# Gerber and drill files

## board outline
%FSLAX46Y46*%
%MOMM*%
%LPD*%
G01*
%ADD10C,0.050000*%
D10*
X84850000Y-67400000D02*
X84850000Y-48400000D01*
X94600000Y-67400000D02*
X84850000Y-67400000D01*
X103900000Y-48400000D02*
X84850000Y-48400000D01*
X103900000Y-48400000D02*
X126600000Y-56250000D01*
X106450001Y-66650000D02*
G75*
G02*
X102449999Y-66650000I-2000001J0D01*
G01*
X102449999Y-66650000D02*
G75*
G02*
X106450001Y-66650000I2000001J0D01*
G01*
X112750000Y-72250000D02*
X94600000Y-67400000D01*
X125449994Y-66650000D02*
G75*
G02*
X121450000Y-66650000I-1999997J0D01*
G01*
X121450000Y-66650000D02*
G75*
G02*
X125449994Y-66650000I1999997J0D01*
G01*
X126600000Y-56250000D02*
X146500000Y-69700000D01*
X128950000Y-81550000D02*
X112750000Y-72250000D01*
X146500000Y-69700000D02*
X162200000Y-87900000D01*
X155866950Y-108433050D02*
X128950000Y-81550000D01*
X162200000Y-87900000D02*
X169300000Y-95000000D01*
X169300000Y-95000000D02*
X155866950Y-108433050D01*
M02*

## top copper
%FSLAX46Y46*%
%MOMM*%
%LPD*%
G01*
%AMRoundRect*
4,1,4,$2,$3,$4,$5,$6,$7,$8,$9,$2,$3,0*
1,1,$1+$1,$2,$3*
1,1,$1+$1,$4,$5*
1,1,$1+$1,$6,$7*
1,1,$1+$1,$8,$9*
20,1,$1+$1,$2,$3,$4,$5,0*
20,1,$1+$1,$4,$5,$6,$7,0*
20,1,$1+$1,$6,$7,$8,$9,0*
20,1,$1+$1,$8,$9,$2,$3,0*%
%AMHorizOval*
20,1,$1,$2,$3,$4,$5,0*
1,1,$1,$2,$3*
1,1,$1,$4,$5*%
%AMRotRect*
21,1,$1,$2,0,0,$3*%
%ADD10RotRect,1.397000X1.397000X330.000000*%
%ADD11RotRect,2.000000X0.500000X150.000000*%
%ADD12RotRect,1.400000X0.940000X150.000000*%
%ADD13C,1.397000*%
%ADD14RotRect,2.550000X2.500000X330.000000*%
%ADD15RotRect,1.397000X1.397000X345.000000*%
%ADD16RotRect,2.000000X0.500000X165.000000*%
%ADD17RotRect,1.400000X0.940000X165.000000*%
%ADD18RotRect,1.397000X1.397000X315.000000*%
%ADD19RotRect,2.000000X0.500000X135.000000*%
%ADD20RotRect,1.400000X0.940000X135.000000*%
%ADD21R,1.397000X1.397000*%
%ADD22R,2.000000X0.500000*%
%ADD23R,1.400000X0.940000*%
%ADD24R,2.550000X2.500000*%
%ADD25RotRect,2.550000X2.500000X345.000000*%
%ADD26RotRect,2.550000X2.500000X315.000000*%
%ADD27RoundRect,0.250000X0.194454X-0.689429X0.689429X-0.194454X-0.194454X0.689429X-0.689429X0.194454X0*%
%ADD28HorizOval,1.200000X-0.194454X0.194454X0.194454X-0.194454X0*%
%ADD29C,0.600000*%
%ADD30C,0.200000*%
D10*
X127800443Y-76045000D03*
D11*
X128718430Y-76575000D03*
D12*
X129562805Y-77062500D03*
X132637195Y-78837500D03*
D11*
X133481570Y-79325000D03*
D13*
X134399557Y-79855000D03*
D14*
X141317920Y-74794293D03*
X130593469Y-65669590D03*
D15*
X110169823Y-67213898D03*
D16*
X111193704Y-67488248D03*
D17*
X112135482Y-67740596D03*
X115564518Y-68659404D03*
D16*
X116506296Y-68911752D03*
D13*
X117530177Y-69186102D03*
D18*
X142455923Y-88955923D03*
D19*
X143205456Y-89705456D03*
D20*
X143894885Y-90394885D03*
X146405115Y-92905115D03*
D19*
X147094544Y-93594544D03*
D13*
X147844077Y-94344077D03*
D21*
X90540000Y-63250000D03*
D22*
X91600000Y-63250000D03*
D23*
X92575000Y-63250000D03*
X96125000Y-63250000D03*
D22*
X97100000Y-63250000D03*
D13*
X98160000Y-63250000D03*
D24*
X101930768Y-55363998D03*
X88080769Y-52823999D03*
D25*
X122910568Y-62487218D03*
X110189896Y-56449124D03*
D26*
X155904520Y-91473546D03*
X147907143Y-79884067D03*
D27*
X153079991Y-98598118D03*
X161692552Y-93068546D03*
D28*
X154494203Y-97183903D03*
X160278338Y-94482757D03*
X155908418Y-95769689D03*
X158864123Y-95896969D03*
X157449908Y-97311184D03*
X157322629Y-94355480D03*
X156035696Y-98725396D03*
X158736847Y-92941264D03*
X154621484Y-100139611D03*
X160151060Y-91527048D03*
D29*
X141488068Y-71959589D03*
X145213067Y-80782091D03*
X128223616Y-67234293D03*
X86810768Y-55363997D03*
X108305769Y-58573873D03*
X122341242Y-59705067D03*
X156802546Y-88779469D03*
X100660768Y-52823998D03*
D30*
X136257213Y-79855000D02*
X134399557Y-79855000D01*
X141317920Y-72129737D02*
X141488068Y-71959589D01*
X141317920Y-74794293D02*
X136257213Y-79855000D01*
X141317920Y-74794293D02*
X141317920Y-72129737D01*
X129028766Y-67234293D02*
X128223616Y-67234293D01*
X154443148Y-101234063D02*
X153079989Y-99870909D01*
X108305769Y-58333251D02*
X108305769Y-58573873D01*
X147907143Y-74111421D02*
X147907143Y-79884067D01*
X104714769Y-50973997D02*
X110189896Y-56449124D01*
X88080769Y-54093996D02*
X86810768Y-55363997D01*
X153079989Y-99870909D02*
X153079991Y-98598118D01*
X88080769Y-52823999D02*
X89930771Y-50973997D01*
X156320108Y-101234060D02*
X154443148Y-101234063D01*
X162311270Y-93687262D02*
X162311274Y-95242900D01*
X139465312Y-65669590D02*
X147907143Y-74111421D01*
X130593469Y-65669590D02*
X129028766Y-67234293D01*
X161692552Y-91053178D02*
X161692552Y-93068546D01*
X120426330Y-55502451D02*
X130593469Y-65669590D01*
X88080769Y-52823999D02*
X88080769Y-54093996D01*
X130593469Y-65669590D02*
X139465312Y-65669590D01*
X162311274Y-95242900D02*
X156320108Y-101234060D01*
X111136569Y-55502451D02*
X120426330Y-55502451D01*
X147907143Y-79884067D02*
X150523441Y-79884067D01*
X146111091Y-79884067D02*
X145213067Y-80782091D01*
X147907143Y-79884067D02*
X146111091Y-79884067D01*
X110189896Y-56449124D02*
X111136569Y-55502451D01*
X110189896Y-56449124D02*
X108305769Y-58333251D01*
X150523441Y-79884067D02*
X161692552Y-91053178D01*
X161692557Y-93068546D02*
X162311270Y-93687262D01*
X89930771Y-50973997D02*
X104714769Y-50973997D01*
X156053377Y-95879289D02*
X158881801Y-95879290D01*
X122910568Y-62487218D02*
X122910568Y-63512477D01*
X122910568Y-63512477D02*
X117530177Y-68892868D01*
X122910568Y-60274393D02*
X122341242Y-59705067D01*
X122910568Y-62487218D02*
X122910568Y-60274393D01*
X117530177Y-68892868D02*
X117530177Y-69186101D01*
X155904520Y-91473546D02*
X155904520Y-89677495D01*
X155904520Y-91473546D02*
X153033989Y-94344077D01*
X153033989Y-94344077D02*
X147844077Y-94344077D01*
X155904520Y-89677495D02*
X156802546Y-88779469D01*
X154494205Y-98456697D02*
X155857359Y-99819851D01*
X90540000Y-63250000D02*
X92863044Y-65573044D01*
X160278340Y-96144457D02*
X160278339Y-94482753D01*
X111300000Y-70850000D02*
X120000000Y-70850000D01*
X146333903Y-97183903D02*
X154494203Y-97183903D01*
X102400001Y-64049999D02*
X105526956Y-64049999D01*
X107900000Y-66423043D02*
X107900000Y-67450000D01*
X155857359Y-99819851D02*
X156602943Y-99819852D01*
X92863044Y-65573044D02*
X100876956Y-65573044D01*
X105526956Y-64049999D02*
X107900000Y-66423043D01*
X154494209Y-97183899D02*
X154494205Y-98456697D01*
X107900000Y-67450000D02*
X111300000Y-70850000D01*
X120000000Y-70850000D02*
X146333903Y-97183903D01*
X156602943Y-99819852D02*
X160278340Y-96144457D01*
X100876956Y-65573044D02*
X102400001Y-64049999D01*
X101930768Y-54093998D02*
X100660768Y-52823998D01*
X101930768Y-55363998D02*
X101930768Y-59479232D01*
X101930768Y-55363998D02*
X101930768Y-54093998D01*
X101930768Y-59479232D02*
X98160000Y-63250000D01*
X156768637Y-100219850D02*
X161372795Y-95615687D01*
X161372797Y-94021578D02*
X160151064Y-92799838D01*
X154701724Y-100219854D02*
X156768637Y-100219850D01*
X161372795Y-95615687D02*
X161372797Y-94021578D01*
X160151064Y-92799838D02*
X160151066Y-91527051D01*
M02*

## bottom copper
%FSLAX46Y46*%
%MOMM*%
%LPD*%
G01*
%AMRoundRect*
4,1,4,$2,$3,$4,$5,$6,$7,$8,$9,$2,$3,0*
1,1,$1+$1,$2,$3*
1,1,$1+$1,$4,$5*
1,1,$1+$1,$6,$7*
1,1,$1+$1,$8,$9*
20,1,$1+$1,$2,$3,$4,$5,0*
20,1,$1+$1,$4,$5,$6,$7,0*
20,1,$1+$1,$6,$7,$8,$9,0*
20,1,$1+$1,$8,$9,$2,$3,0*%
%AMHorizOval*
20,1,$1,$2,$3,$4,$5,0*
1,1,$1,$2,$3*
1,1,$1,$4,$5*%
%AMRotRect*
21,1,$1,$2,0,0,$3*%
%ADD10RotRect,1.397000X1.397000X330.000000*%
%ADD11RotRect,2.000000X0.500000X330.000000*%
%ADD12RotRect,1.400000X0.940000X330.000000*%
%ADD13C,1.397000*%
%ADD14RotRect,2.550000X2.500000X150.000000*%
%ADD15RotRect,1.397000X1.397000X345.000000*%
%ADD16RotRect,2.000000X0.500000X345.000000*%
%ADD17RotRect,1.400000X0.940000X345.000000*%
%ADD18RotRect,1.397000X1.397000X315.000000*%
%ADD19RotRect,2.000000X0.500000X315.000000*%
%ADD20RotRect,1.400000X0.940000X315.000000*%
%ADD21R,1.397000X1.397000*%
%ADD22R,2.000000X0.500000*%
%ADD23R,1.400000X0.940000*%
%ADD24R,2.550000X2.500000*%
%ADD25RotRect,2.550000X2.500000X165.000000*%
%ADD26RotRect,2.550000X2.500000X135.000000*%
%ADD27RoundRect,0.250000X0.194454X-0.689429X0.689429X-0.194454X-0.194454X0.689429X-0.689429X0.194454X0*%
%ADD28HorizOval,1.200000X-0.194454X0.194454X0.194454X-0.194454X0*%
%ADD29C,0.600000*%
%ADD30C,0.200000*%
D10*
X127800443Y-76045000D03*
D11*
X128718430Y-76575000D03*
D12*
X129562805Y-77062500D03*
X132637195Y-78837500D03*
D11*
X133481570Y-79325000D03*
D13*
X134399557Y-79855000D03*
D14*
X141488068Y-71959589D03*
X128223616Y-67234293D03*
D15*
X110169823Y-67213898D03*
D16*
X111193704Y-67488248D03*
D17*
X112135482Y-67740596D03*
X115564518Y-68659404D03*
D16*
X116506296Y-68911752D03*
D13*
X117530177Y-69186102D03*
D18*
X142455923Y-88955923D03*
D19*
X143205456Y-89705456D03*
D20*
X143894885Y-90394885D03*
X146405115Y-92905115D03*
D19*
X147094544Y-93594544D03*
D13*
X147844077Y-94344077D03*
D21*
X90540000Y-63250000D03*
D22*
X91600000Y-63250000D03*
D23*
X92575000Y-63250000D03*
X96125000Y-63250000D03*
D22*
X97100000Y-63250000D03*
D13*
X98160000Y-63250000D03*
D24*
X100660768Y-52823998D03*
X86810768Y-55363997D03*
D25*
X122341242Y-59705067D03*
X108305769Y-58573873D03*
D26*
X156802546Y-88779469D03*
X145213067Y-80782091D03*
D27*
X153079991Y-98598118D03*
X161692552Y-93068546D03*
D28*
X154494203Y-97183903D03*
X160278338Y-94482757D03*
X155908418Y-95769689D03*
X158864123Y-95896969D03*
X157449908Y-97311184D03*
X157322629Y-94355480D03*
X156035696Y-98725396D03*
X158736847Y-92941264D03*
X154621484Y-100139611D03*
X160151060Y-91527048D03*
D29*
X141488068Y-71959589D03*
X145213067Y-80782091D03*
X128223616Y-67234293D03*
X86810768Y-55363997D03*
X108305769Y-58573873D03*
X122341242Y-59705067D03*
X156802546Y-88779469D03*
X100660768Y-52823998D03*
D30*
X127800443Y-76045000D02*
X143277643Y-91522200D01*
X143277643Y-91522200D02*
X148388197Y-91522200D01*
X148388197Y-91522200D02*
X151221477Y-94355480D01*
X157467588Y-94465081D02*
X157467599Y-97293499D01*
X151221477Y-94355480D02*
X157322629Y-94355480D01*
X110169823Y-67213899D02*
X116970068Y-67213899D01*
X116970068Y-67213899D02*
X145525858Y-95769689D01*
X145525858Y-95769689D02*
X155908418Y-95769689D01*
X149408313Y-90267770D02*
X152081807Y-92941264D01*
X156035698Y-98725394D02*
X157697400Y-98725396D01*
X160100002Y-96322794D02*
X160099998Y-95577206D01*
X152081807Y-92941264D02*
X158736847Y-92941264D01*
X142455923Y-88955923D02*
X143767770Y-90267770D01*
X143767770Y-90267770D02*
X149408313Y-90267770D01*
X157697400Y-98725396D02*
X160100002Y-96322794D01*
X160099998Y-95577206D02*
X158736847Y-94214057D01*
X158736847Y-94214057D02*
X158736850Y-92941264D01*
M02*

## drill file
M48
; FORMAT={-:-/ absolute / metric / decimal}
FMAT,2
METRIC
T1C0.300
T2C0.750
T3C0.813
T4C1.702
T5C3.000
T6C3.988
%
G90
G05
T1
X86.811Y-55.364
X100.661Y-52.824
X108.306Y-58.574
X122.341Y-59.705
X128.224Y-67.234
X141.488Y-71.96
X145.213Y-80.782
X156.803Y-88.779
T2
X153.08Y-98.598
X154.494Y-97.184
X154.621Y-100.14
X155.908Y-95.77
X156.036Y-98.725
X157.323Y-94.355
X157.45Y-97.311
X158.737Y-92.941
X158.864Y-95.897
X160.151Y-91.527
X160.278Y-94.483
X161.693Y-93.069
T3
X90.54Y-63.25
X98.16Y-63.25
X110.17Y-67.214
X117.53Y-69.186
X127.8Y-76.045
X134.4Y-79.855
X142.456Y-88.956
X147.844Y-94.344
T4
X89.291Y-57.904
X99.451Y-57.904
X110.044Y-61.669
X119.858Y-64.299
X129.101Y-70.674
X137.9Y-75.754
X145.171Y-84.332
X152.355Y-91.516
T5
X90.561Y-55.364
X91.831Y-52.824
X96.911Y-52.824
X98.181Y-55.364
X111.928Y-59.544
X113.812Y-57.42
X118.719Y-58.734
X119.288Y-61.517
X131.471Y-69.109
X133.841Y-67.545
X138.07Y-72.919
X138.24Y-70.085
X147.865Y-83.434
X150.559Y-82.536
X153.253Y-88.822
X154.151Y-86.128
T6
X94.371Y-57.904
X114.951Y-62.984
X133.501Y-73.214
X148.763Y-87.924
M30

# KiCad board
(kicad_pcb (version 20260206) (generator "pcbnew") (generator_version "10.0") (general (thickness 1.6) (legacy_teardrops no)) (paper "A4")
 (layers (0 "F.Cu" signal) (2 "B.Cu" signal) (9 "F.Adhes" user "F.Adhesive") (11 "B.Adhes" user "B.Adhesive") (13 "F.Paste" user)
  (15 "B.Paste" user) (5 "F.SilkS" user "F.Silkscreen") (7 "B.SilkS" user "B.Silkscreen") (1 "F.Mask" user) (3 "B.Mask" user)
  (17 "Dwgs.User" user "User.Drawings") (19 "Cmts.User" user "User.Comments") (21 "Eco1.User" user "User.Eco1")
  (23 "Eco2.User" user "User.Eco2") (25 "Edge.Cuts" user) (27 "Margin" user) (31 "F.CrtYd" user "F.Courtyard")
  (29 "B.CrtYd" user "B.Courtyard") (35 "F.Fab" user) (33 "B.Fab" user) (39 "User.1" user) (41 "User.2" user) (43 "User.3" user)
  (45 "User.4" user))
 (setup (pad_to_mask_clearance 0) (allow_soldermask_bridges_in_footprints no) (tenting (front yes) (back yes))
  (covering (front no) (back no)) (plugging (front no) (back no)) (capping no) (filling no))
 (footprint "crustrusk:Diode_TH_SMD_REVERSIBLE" (layer "F.Cu") (at 131.1 77.95 -30)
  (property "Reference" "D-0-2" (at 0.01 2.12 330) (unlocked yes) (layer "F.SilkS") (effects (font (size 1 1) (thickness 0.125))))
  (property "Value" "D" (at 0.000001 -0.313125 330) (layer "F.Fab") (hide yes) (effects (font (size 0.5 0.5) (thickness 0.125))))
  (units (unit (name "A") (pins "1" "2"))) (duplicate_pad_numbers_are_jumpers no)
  (pad "1" thru_hole rect (at -3.81 0 330) (size 1.397 1.397) (drill 0.8128) (layers "*.Cu" "*.Mask") (remove_unused_layers no)
   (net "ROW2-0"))
  (pad "1" smd rect (at -2.75 0 150) (size 2 0.5) (layers "F.Cu") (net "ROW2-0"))
  (pad "1" smd rect (at -2.75 0 330) (size 2 0.5) (layers "B.Cu") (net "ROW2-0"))
  (pad "1" smd rect (at -1.775 0 150) (size 1.4 0.94) (layers "F.Cu" "F.Mask" "F.Paste") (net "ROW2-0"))
  (pad "1" smd rect (at -1.775 0 330) (size 1.4 0.94) (layers "B.Cu" "B.Mask" "B.Paste") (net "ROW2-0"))
  (pad "2" smd rect (at 1.775 0 150) (size 1.4 0.94) (layers "F.Cu" "F.Mask" "F.Paste") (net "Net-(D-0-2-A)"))
  (pad "2" smd rect (at 1.775 0 330) (size 1.4 0.94) (layers "B.Cu" "B.Mask" "B.Paste") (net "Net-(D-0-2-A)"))
  (pad "2" smd rect (at 2.75 0 150) (size 2 0.5) (layers "F.Cu") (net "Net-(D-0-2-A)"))
  (pad "2" smd rect (at 2.75 0 330) (size 2 0.5) (layers "B.Cu") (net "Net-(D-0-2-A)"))
  (pad "2" thru_hole circle (at 3.81 0 330) (size 1.397 1.397) (drill 0.8128) (layers "*.Cu" "*.Mask") (remove_unused_layers no)
   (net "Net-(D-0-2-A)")))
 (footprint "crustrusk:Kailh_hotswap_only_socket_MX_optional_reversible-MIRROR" (layer "F.Cu") (at 133.500768 73.213998 -30)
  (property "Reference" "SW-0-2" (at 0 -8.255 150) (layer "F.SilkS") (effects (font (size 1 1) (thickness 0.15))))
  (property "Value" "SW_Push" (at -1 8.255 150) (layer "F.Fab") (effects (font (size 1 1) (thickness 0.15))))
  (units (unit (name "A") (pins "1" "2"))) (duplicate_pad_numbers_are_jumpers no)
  (pad "" np_thru_hole circle (at -5.08 0 330) (size 1.7018 1.7018) (drill 1.7018) (layers "*.Cu" "*.Mask"))
  (pad "" np_thru_hole circle (at -3.81 -2.54 150) (size 3 3) (drill 3) (layers "*.Cu" "*.Mask"))
  (pad "" np_thru_hole circle (at -2.54 -5.079997 330) (size 3 3) (drill 3) (layers "*.Cu" "*.Mask"))
  (pad "" np_thru_hole circle (at 0 0 330) (size 3.9878 3.9878) (drill 3.9878) (layers "*.Cu" "*.Mask"))
  (pad "" np_thru_hole circle (at 2.540002 -5.080001 150) (size 3 3) (drill 3) (layers "*.Cu" "*.Mask"))
  (pad "" np_thru_hole circle (at 3.81 -2.540001 330) (size 3 3) (drill 3) (layers "*.Cu" "*.Mask"))
  (pad "" np_thru_hole circle (at 5.08 0 330) (size 1.7018 1.7018) (drill 1.7018) (layers "*.Cu" "*.Mask"))
  (pad "1" smd rect (at 6.29 -5.08 150) (size 2.55 2.5) (layers "B.Cu" "B.Mask" "B.Paste") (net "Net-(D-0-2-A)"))
  (pad "1" smd rect (at 7.56 -2.54 330) (size 2.55 2.5) (layers "F.Cu" "F.Mask" "F.Paste") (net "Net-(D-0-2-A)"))
  (pad "2" smd rect (at -7.56 -2.54 150) (size 2.55 2.5) (layers "B.Cu" "B.Mask" "B.Paste") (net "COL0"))
  (pad "2" smd rect (at -6.289999 -5.079999 330) (size 2.55 2.5) (layers "F.Cu" "F.Mask" "F.Paste") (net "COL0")))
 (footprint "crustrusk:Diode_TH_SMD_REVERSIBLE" (layer "F.Cu") (at 113.85 68.2 -15)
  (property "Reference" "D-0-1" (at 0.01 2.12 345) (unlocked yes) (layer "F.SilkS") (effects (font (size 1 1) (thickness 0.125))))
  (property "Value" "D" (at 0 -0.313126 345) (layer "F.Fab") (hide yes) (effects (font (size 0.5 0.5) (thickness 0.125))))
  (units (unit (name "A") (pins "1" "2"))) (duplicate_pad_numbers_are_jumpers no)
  (pad "1" thru_hole rect (at -3.81 -0.000001 345) (size 1.397 1.397) (drill 0.8128) (layers "*.Cu" "*.Mask") (remove_unused_layers no)
   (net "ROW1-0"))
  (pad "1" smd rect (at -2.75 0 165) (size 2 0.5) (layers "F.Cu") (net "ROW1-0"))
  (pad "1" smd rect (at -2.75 0 345) (size 2 0.5) (layers "B.Cu") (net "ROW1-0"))
  (pad "1" smd rect (at -1.775 0 165) (size 1.4 0.94) (layers "F.Cu" "F.Mask" "F.Paste") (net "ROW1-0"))
  (pad "1" smd rect (at -1.775 0 345) (size 1.4 0.94) (layers "B.Cu" "B.Mask" "B.Paste") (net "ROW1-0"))
  (pad "2" smd rect (at 1.775 0 165) (size 1.4 0.94) (layers "F.Cu" "F.Mask" "F.Paste") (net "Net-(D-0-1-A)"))
  (pad "2" smd rect (at 1.775 0 345) (size 1.4 0.94) (layers "B.Cu" "B.Mask" "B.Paste") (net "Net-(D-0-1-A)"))
  (pad "2" smd rect (at 2.75 0 165) (size 2 0.5) (layers "F.Cu") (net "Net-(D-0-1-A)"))
  (pad "2" smd rect (at 2.75 0 345) (size 2 0.5) (layers "B.Cu") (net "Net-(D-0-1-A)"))
  (pad "2" thru_hole circle (at 3.81 0.000001 345) (size 1.397 1.397) (drill 0.8128) (layers "*.Cu" "*.Mask") (remove_unused_layers no)
   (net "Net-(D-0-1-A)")))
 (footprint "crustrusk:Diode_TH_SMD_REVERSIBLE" (layer "F.Cu") (at 145.15 91.65 -45)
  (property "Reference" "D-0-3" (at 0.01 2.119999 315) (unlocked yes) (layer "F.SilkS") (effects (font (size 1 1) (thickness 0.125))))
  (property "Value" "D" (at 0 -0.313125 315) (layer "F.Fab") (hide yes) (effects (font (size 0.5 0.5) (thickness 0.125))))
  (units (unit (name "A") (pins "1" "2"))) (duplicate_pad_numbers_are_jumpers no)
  (pad "1" thru_hole rect (at -3.81 0 315) (size 1.397 1.397) (drill 0.8128) (layers "*.Cu" "*.Mask") (remove_unused_layers no)
   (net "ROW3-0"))
  (pad "1" smd rect (at -2.75 0 135) (size 2 0.5) (layers "F.Cu") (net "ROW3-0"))
  (pad "1" smd rect (at -2.75 0 315) (size 2 0.5) (layers "B.Cu") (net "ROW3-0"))
  (pad "1" smd rect (at -1.775001 0 135) (size 1.4 0.94) (layers "F.Cu" "F.Mask" "F.Paste") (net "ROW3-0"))
  (pad "1" smd rect (at -1.775001 0 315) (size 1.4 0.94) (layers "B.Cu" "B.Mask" "B.Paste") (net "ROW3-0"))
  (pad "2" smd rect (at 1.775001 0 135) (size 1.4 0.94) (layers "F.Cu" "F.Mask" "F.Paste") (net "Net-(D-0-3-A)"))
  (pad "2" smd rect (at 1.775001 0 315) (size 1.4 0.94) (layers "B.Cu" "B.Mask" "B.Paste") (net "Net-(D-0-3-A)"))
  (pad "2" smd rect (at 2.75 0 135) (size 2 0.5) (layers "F.Cu") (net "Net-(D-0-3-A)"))
  (pad "2" smd rect (at 2.75 0 315) (size 2 0.5) (layers "B.Cu") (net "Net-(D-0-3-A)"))
  (pad "2" thru_hole circle (at 3.81 0 315) (size 1.397 1.397) (drill 0.8128) (layers "*.Cu" "*.Mask") (remove_unused_layers no)
   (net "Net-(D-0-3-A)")))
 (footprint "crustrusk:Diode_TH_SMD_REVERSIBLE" (layer "F.Cu") (at 94.35 63.25)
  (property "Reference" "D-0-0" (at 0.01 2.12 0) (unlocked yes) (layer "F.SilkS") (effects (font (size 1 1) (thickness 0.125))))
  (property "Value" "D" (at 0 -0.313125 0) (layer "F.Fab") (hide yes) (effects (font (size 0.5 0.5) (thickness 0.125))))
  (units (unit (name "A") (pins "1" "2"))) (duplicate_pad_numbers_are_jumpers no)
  (pad "1" thru_hole rect (at -3.81 0) (size 1.397 1.397) (drill 0.8128) (layers "*.Cu" "*.Mask") (remove_unused_layers no) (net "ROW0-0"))
  (pad "1" smd rect (at -2.75 0 180) (size 2 0.5) (layers "F.Cu") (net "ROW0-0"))
  (pad "1" smd rect (at -2.75 0) (size 2 0.5) (layers "B.Cu") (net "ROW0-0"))
  (pad "1" smd rect (at -1.775 0 180) (size 1.4 0.94) (layers "F.Cu" "F.Mask" "F.Paste") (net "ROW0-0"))
  (pad "1" smd rect (at -1.775 0) (size 1.4 0.94) (layers "B.Cu" "B.Mask" "B.Paste") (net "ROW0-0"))
  (pad "2" smd rect (at 1.775 0 180) (size 1.4 0.94) (layers "F.Cu" "F.Mask" "F.Paste") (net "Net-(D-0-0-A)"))
  (pad "2" smd rect (at 1.775 0) (size 1.4 0.94) (layers "B.Cu" "B.Mask" "B.Paste") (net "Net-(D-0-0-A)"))
  (pad "2" smd rect (at 2.75 0 180) (size 2 0.5) (layers "F.Cu") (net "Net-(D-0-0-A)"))
  (pad "2" smd rect (at 2.75 0) (size 2 0.5) (layers "B.Cu") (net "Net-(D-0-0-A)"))
  (pad "2" thru_hole circle (at 3.81 0) (size 1.397 1.397) (drill 0.8128) (layers "*.Cu" "*.Mask") (remove_unused_layers no)
   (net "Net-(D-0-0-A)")))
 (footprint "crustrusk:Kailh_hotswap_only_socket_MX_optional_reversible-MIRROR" (layer "F.Cu") (at 94.370768 57.903998)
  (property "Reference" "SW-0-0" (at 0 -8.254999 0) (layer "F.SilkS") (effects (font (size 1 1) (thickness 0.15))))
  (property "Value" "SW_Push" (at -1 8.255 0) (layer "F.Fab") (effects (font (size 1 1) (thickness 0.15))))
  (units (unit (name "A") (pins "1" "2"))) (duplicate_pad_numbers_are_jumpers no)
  (pad "" np_thru_hole circle (at -5.079999 0) (size 1.7018 1.7018) (drill 1.7018) (layers "*.Cu" "*.Mask"))
  (pad "" np_thru_hole circle (at -3.81 -2.54 180) (size 3 3) (drill 3) (layers "*.Cu" "*.Mask"))
  (pad "" np_thru_hole circle (at -2.54 -5.079998) (size 3 3) (drill 3) (layers "*.Cu" "*.Mask"))
  (pad "" np_thru_hole circle (at 0 0) (size 3.9878 3.9878) (drill 3.9878) (layers "*.Cu" "*.Mask"))
  (pad "" np_thru_hole circle (at 2.540002 -5.080001 180) (size 3 3) (drill 3) (layers "*.Cu" "*.Mask"))
  (pad "" np_thru_hole circle (at 3.81 -2.54) (size 3 3) (drill 3) (layers "*.Cu" "*.Mask"))
  (pad "" np_thru_hole circle (at 5.079999 0) (size 1.7018 1.7018) (drill 1.7018) (layers "*.Cu" "*.Mask"))
  (pad "1" smd rect (at 6.29 -5.08 180) (size 2.55 2.5) (layers "B.Cu" "B.Mask" "B.Paste") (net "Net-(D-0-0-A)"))
  (pad "1" smd rect (at 7.56 -2.54) (size 2.55 2.5) (layers "F.Cu" "F.Mask" "F.Paste") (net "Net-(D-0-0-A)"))
  (pad "2" smd rect (at -7.56 -2.540001 180) (size 2.55 2.5) (layers "B.Cu" "B.Mask" "B.Paste") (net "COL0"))
  (pad "2" smd rect (at -6.289999 -5.079999) (size 2.55 2.5) (layers "F.Cu" "F.Mask" "F.Paste") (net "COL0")))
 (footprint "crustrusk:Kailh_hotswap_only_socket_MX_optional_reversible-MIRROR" (layer "F.Cu") (at 114.950768 62.983998 -15)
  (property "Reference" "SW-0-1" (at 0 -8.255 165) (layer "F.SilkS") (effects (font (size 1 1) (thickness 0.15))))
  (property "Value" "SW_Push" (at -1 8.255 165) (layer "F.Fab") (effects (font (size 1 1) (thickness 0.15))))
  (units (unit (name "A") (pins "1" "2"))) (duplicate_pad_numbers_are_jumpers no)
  (pad "" np_thru_hole circle (at -5.08 0 345) (size 1.7018 1.7018) (drill 1.7018) (layers "*.Cu" "*.Mask"))
  (pad "" np_thru_hole circle (at -3.810001 -2.54 165) (size 3 3) (drill 3) (layers "*.Cu" "*.Mask"))
  (pad "" np_thru_hole circle (at -2.54 -5.079998 345) (size 3 3) (drill 3) (layers "*.Cu" "*.Mask"))
  (pad "" np_thru_hole circle (at 0 0 345) (size 3.9878 3.9878) (drill 3.9878) (layers "*.Cu" "*.Mask"))
  (pad "" np_thru_hole circle (at 2.540003 -5.080001 165) (size 3 3) (drill 3) (layers "*.Cu" "*.Mask"))
  (pad "" np_thru_hole circle (at 3.81 -2.54 345) (size 3 3) (drill 3) (layers "*.Cu" "*.Mask"))
  (pad "" np_thru_hole circle (at 5.08 0 345) (size 1.7018 1.7018) (drill 1.7018) (layers "*.Cu" "*.Mask"))
  (pad "1" smd rect (at 6.29 -5.08 165) (size 2.55 2.5) (layers "B.Cu" "B.Mask" "B.Paste") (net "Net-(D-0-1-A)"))
  (pad "1" smd rect (at 7.56 -2.54 345) (size 2.55 2.5) (layers "F.Cu" "F.Mask" "F.Paste") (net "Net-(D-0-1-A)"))
  (pad "2" smd rect (at -7.56 -2.540001 165) (size 2.55 2.5) (layers "B.Cu" "B.Mask" "B.Paste") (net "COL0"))
  (pad "2" smd rect (at -6.289999 -5.079999 345) (size 2.55 2.5) (layers "F.Cu" "F.Mask" "F.Paste") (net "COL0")))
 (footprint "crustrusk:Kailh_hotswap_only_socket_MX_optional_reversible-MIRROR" (layer "F.Cu") (at 148.762742 87.92387 -45)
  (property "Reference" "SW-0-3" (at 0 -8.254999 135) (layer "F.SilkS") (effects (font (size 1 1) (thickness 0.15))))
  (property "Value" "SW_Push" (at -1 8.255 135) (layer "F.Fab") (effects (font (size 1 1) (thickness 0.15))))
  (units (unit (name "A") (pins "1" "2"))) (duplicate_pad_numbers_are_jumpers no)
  (pad "" np_thru_hole circle (at -5.079999 0 315) (size 1.7018 1.7018) (drill 1.7018) (layers "*.Cu" "*.Mask"))
  (pad "" np_thru_hole circle (at -3.81 -2.54 135) (size 3 3) (drill 3) (layers "*.Cu" "*.Mask"))
  (pad "" np_thru_hole circle (at -2.54 -5.079998 315) (size 3 3) (drill 3) (layers "*.Cu" "*.Mask"))
  (pad "" np_thru_hole circle (at 0 0 315) (size 3.9878 3.9878) (drill 3.9878) (layers "*.Cu" "*.Mask"))
  (pad "" np_thru_hole circle (at 2.540002 -5.080001 135) (size 3 3) (drill 3) (layers "*.Cu" "*.Mask"))
  (pad "" np_thru_hole circle (at 3.81 -2.54 315) (size 3 3) (drill 3) (layers "*.Cu" "*.Mask"))
  (pad "" np_thru_hole circle (at 5.079999 0 315) (size 1.7018 1.7018) (drill 1.7018) (layers "*.Cu" "*.Mask"))
  (pad "1" smd rect (at 6.29 -5.08 135) (size 2.55 2.5) (layers "B.Cu" "B.Mask" "B.Paste") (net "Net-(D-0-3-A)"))
  (pad "1" smd rect (at 7.56 -2.54 315) (size 2.55 2.5) (layers "F.Cu" "F.Mask" "F.Paste") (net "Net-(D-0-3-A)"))
  (pad "2" smd rect (at -7.56 -2.540001 135) (size 2.55 2.5) (layers "B.Cu" "B.Mask" "B.Paste") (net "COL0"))
  (pad "2" smd rect (at -6.289999 -5.079999 315) (size 2.55 2.5) (layers "F.Cu" "F.Mask" "F.Paste") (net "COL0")))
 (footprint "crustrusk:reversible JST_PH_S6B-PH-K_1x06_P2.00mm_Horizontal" (layer "F.Cu") (at 153.079991 98.598118 45)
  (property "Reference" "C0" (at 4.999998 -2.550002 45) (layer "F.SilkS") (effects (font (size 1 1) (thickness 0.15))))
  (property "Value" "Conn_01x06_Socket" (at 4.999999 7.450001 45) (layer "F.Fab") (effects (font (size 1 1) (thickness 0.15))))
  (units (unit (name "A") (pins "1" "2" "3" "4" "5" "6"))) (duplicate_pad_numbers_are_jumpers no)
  (pad "1" thru_hole roundrect (at 0 0 45) (size 1.2 1.75) (drill 0.75) (layers "*.Cu" "*.Mask") (remove_unused_layers no)
   (roundrect_rratio 0.208333) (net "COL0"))
  (pad "1" thru_hole roundrect (at 9.999998 2.180002 45) (size 1.2 1.75) (drill 0.75) (layers "*.Cu" "*.Mask") (remove_unused_layers no)
   (roundrect_rratio 0.208333) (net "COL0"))
  (pad "2" thru_hole oval (at 2 -0.000002 45) (size 1.2 1.75) (drill 0.75) (layers "*.Cu" "*.Mask") (remove_unused_layers no) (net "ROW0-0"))
  (pad "2" thru_hole oval (at 8 2.18 45) (size 1.2 1.75) (drill 0.75) (layers "*.Cu" "*.Mask") (remove_unused_layers no) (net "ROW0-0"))
  (pad "3" thru_hole oval (at 4.000001 -0.000001 45) (size 1.2 1.75) (drill 0.75) (layers "*.Cu" "*.Mask") (remove_unused_layers no)
   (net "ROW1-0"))
  (pad "3" thru_hole oval (at 6 2.179998 45) (size 1.2 1.75) (drill 0.75) (layers "*.Cu" "*.Mask") (remove_unused_layers no) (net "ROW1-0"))
  (pad "4" thru_hole oval (at 3.999998 2.179998 45) (size 1.2 1.75) (drill 0.75) (layers "*.Cu" "*.Mask") (remove_unused_layers no)
   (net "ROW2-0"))
  (pad "4" thru_hole oval (at 5.999996 0 45) (size 1.2 1.75) (drill 0.75) (layers "*.Cu" "*.Mask") (remove_unused_layers no) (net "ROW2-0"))
  (pad "5" thru_hole oval (at 2 2.179998 45) (size 1.2 1.75) (drill 0.75) (layers "*.Cu" "*.Mask") (remove_unused_layers no) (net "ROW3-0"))
  (pad "5" thru_hole oval (at 8.000001 0.000001 45) (size 1.2 1.75) (drill 0.75) (layers "*.Cu" "*.Mask") (remove_unused_layers no)
   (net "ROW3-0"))
  (pad "6" thru_hole oval (at 0 2.18 45) (size 1.2 1.75) (drill 0.75) (layers "*.Cu" "*.Mask") (remove_unused_layers no) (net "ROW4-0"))
  (pad "6" thru_hole oval (at 10.000002 -0.000001 45) (size 1.2 1.75) (drill 0.75) (layers "*.Cu" "*.Mask") (remove_unused_layers no)
   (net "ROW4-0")))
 (gr_line (start 84.85 67.4) (end 84.85 48.4) (stroke (width 0.05) (type default)) (layer "Edge.Cuts"))
 (gr_line (start 94.6 67.4) (end 84.85 67.4) (stroke (width 0.05) (type default)) (layer "Edge.Cuts"))
 (gr_line (start 103.9 48.4) (end 84.85 48.4) (stroke (width 0.05) (type default)) (layer "Edge.Cuts"))
 (gr_line (start 103.9 48.4) (end 126.6 56.25) (stroke (width 0.05) (type default)) (layer "Edge.Cuts"))
 (gr_circle (center 104.45 66.65) (end 102.449999 66.65) (stroke (width 0.05) (type default)) (fill no) (layer "Edge.Cuts"))
 (gr_line (start 112.75 72.25) (end 94.6 67.4) (stroke (width 0.05) (type default)) (layer "Edge.Cuts"))
 (gr_circle (center 123.449997 66.65) (end 121.45 66.65) (stroke (width 0.05) (type default)) (fill no) (layer "Edge.Cuts"))
 (gr_line (start 126.6 56.25) (end 146.5 69.7) (stroke (width 0.05) (type default)) (layer "Edge.Cuts"))
 (gr_line (start 128.95 81.55) (end 112.75 72.25) (stroke (width 0.05) (type default)) (layer "Edge.Cuts"))
 (gr_line (start 146.5 69.7) (end 162.2 87.9) (stroke (width 0.05) (type default)) (layer "Edge.Cuts"))
 (gr_line (start 155.86695 108.43305) (end 128.95 81.55) (stroke (width 0.05) (type default)) (layer "Edge.Cuts"))
 (gr_line (start 162.2 87.9) (end 169.3 95) (stroke (width 0.05) (type default)) (layer "Edge.Cuts"))
 (gr_line (start 169.3 95) (end 155.86695 108.43305) (stroke (width 0.05) (type default)) (layer "Edge.Cuts"))
 (segment (start 127.800443 76.045) (end 143.277643 91.5222) (width 0.2) (layer "B.Cu") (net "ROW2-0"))
 (segment (start 143.277643 91.5222) (end 148.388197 91.5222) (width 0.2) (layer "B.Cu") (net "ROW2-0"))
 (segment (start 148.388197 91.5222) (end 151.221477 94.35548) (width 0.2) (layer "B.Cu") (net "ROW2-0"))
 (segment (start 157.467588 94.465081) (end 157.467599 97.293499) (width 0.2) (layer "B.Cu") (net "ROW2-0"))
 (segment (start 151.221477 94.35548) (end 157.322629 94.35548) (width 0.2) (layer "B.Cu") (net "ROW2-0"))
 (segment (start 136.257213 79.855) (end 134.399557 79.855) (width 0.2) (layer "F.Cu") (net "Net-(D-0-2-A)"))
 (segment (start 141.31792 72.129737) (end 141.488068 71.959589) (width 0.2) (layer "F.Cu") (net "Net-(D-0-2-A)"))
 (segment (start 141.31792 74.794293) (end 136.257213 79.855) (width 0.2) (layer "F.Cu") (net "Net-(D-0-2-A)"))
 (segment (start 141.31792 74.794293) (end 141.31792 72.129737) (width 0.2) (layer "F.Cu") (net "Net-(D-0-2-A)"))
 (via (at 141.488068 71.959589) (size 0.6) (drill 0.3) (layers "F.Cu" "B.Cu") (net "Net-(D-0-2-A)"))
 (segment (start 129.028766 67.234293) (end 128.223616 67.234293) (width 0.2) (layer "F.Cu") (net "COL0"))
 (segment (start 154.443148 101.234063) (end 153.079989 99.870909) (width 0.2) (layer "F.Cu") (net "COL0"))
 (segment (start 108.305769 58.333251) (end 108.305769 58.573873) (width 0.2) (layer "F.Cu") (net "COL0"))
 (segment (start 147.907143 74.111421) (end 147.907143 79.884067) (width 0.2) (layer "F.Cu") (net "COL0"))
 (segment (start 104.714769 50.973997) (end 110.189896 56.449124) (width 0.2) (layer "F.Cu") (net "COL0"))
 (segment (start 88.080769 54.093996) (end 86.810768 55.363997) (width 0.2) (layer "F.Cu") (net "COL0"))
 (segment (start 153.079989 99.870909) (end 153.079991 98.598118) (width 0.2) (layer "F.Cu") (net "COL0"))
 (segment (start 88.080769 52.823999) (end 89.930771 50.973997) (width 0.2) (layer "F.Cu") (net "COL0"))
 (segment (start 156.320108 101.23406) (end 154.443148 101.234063) (width 0.2) (layer "F.Cu") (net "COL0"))
 (segment (start 162.31127 93.687262) (end 162.311274 95.2429) (width 0.2) (layer "F.Cu") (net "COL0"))
 (segment (start 139.465312 65.66959) (end 147.907143 74.111421) (width 0.2) (layer "F.Cu") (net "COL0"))
 (segment (start 130.593469 65.66959) (end 129.028766 67.234293) (width 0.2) (layer "F.Cu") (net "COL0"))
 (segment (start 161.692552 91.053178) (end 161.692552 93.068546) (width 0.2) (layer "F.Cu") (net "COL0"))
 (segment (start 120.42633 55.502451) (end 130.593469 65.66959) (width 0.2) (layer "F.Cu") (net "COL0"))
 (segment (start 88.080769 52.823999) (end 88.080769 54.093996) (width 0.2) (layer "F.Cu") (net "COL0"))
 (segment (start 130.593469 65.66959) (end 139.465312 65.66959) (width 0.2) (layer "F.Cu") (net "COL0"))
 (segment (start 162.311274 95.2429) (end 156.320108 101.23406) (width 0.2) (layer "F.Cu") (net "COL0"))
 (segment (start 111.136569 55.502451) (end 120.42633 55.502451) (width 0.2) (layer "F.Cu") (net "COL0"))
 (segment (start 147.907143 79.884067) (end 150.523441 79.884067) (width 0.2) (layer "F.Cu") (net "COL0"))
 (segment (start 146.111091 79.884067) (end 145.213067 80.782091) (width 0.2) (layer "F.Cu") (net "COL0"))
 (segment (start 147.907143 79.884067) (end 146.111091 79.884067) (width 0.2) (layer "F.Cu") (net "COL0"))
 (segment (start 110.189896 56.449124) (end 111.136569 55.502451) (width 0.2) (layer "F.Cu") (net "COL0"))
 (segment (start 110.189896 56.449124) (end 108.305769 58.333251) (width 0.2) (layer "F.Cu") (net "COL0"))
 (segment (start 150.523441 79.884067) (end 161.692552 91.053178) (width 0.2) (layer "F.Cu") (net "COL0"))
 (segment (start 161.692557 93.068546) (end 162.31127 93.687262) (width 0.2) (layer "F.Cu") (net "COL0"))
 (segment (start 89.930771 50.973997) (end 104.714769 50.973997) (width 0.2) (layer "F.Cu") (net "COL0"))
 (via (at 145.213067 80.782091) (size 0.6) (drill 0.3) (layers "F.Cu" "B.Cu") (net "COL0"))
 (via (at 128.223616 67.234293) (size 0.6) (drill 0.3) (layers "F.Cu" "B.Cu") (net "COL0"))
 (via (at 86.810768 55.363997) (size 0.6) (drill 0.3) (layers "F.Cu" "B.Cu") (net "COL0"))
 (via (at 108.305769 58.573873) (size 0.6) (drill 0.3) (layers "F.Cu" "B.Cu") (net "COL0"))
 (segment (start 156.053377 95.879289) (end 158.881801 95.87929) (width 0.2) (layer "F.Cu") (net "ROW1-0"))
 (segment (start 110.169823 67.213899) (end 116.970068 67.213899) (width 0.2) (layer "B.Cu") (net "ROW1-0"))
 (segment (start 116.970068 67.213899) (end 145.525858 95.769689) (width 0.2) (layer "B.Cu") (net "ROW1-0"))
 (segment (start 145.525858 95.769689) (end 155.908418 95.769689) (width 0.2) (layer "B.Cu") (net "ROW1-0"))
 (segment (start 122.910568 62.487218) (end 122.910568 63.512477) (width 0.2) (layer "F.Cu") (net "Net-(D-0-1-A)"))
 (segment (start 122.910568 63.512477) (end 117.530177 68.892868) (width 0.2) (layer "F.Cu") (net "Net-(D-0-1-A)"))
 (segment (start 122.910568 60.274393) (end 122.341242 59.705067) (width 0.2) (layer "F.Cu") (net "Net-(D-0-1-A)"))
 (segment (start 122.910568 62.487218) (end 122.910568 60.274393) (width 0.2) (layer "F.Cu") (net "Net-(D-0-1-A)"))
 (segment (start 117.530177 68.892868) (end 117.530177 69.186101) (width 0.2) (layer "F.Cu") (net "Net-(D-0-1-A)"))
 (via (at 122.341242 59.705067) (size 0.6) (drill 0.3) (layers "F.Cu" "B.Cu") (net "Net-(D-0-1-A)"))
 (segment (start 149.408313 90.26777) (end 152.081807 92.941264) (width 0.2) (layer "B.Cu") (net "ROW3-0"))
 (segment (start 156.035698 98.725394) (end 157.6974 98.725396) (width 0.2) (layer "B.Cu") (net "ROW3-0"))
 (segment (start 160.100002 96.322794) (end 160.099998 95.577206) (width 0.2) (layer "B.Cu") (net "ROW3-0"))
 (segment (start 152.081807 92.941264) (end 158.736847 92.941264) (width 0.2) (layer "B.Cu") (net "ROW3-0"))
 (segment (start 142.455923 88.955923) (end 143.76777 90.26777) (width 0.2) (layer "B.Cu") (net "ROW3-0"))
 (segment (start 143.76777 90.26777) (end 149.408313 90.26777) (width 0.2) (layer "B.Cu") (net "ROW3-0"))
 (segment (start 157.6974 98.725396) (end 160.100002 96.322794) (width 0.2) (layer "B.Cu") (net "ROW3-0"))
 (segment (start 160.099998 95.577206) (end 158.736847 94.214057) (width 0.2) (layer "B.Cu") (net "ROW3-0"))
 (segment (start 158.736847 94.214057) (end 158.73685 92.941264) (width 0.2) (layer "B.Cu") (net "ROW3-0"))
 (segment (start 155.90452 91.473546) (end 155.90452 89.677495) (width 0.2) (layer "F.Cu") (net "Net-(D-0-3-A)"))
 (segment (start 155.90452 91.473546) (end 153.033989 94.344077) (width 0.2) (layer "F.Cu") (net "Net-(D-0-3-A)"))
 (segment (start 153.033989 94.344077) (end 147.844077 94.344077) (width 0.2) (layer "F.Cu") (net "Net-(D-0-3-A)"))
 (segment (start 155.90452 89.677495) (end 156.802546 88.779469) (width 0.2) (layer "F.Cu") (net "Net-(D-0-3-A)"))
 (via (at 156.802546 88.779469) (size 0.6) (drill 0.3) (layers "F.Cu" "B.Cu") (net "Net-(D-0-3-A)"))
 (segment (start 154.494205 98.456697) (end 155.857359 99.819851) (width 0.2) (layer "F.Cu") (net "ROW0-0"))
 (segment (start 90.54 63.25) (end 92.863044 65.573044) (width 0.2) (layer "F.Cu") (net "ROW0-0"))
 (segment (start 160.27834 96.144457) (end 160.278339 94.482753) (width 0.2) (layer "F.Cu") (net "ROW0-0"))
 (segment (start 111.3 70.85) (end 120 70.85) (width 0.2) (layer "F.Cu") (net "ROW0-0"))
 (segment (start 146.333903 97.183903) (end 154.494203 97.183903) (width 0.2) (layer "F.Cu") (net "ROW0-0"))
 (segment (start 102.400001 64.049999) (end 105.526956 64.049999) (width 0.2) (layer "F.Cu") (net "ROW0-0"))
 (segment (start 107.9 66.423043) (end 107.9 67.45) (width 0.2) (layer "F.Cu") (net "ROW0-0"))
 (segment (start 155.857359 99.819851) (end 156.602943 99.819852) (width 0.2) (layer "F.Cu") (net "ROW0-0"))
 (segment (start 92.863044 65.573044) (end 100.876956 65.573044) (width 0.2) (layer "F.Cu") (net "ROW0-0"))
 (segment (start 105.526956 64.049999) (end 107.9 66.423043) (width 0.2) (layer "F.Cu") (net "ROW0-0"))
 (segment (start 154.494209 97.183899) (end 154.494205 98.456697) (width 0.2) (layer "F.Cu") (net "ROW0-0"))
 (segment (start 107.9 67.45) (end 111.3 70.85) (width 0.2) (layer "F.Cu") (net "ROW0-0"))
 (segment (start 120 70.85) (end 146.333903 97.183903) (width 0.2) (layer "F.Cu") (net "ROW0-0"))
 (segment (start 156.602943 99.819852) (end 160.27834 96.144457) (width 0.2) (layer "F.Cu") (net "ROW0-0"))
 (segment (start 100.876956 65.573044) (end 102.400001 64.049999) (width 0.2) (layer "F.Cu") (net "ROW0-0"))
 (segment (start 101.930768 54.093998) (end 100.660768 52.823998) (width 0.2) (layer "F.Cu") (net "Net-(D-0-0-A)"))
 (segment (start 101.930768 55.363998) (end 101.930768 59.479232) (width 0.2) (layer "F.Cu") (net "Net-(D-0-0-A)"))
 (segment (start 101.930768 55.363998) (end 101.930768 54.093998) (width 0.2) (layer "F.Cu") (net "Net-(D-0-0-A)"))
 (segment (start 101.930768 59.479232) (end 98.16 63.25) (width 0.2) (layer "F.Cu") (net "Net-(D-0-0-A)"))
 (via (at 100.660768 52.823998) (size 0.6) (drill 0.3) (layers "F.Cu" "B.Cu") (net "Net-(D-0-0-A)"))
 (segment (start 156.768637 100.21985) (end 161.372795 95.615687) (width 0.2) (layer "F.Cu") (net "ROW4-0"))
 (segment (start 161.372797 94.021578) (end 160.151064 92.799838) (width 0.2) (layer "F.Cu") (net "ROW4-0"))
 (segment (start 154.701724 100.219854) (end 156.768637 100.21985) (width 0.2) (layer "F.Cu") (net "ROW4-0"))
 (segment (start 161.372795 95.615687) (end 161.372797 94.021578) (width 0.2) (layer "F.Cu") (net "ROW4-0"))
 (segment (start 160.151064 92.799838) (end 160.151066 91.527051) (width 0.2) (layer "F.Cu") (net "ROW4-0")))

